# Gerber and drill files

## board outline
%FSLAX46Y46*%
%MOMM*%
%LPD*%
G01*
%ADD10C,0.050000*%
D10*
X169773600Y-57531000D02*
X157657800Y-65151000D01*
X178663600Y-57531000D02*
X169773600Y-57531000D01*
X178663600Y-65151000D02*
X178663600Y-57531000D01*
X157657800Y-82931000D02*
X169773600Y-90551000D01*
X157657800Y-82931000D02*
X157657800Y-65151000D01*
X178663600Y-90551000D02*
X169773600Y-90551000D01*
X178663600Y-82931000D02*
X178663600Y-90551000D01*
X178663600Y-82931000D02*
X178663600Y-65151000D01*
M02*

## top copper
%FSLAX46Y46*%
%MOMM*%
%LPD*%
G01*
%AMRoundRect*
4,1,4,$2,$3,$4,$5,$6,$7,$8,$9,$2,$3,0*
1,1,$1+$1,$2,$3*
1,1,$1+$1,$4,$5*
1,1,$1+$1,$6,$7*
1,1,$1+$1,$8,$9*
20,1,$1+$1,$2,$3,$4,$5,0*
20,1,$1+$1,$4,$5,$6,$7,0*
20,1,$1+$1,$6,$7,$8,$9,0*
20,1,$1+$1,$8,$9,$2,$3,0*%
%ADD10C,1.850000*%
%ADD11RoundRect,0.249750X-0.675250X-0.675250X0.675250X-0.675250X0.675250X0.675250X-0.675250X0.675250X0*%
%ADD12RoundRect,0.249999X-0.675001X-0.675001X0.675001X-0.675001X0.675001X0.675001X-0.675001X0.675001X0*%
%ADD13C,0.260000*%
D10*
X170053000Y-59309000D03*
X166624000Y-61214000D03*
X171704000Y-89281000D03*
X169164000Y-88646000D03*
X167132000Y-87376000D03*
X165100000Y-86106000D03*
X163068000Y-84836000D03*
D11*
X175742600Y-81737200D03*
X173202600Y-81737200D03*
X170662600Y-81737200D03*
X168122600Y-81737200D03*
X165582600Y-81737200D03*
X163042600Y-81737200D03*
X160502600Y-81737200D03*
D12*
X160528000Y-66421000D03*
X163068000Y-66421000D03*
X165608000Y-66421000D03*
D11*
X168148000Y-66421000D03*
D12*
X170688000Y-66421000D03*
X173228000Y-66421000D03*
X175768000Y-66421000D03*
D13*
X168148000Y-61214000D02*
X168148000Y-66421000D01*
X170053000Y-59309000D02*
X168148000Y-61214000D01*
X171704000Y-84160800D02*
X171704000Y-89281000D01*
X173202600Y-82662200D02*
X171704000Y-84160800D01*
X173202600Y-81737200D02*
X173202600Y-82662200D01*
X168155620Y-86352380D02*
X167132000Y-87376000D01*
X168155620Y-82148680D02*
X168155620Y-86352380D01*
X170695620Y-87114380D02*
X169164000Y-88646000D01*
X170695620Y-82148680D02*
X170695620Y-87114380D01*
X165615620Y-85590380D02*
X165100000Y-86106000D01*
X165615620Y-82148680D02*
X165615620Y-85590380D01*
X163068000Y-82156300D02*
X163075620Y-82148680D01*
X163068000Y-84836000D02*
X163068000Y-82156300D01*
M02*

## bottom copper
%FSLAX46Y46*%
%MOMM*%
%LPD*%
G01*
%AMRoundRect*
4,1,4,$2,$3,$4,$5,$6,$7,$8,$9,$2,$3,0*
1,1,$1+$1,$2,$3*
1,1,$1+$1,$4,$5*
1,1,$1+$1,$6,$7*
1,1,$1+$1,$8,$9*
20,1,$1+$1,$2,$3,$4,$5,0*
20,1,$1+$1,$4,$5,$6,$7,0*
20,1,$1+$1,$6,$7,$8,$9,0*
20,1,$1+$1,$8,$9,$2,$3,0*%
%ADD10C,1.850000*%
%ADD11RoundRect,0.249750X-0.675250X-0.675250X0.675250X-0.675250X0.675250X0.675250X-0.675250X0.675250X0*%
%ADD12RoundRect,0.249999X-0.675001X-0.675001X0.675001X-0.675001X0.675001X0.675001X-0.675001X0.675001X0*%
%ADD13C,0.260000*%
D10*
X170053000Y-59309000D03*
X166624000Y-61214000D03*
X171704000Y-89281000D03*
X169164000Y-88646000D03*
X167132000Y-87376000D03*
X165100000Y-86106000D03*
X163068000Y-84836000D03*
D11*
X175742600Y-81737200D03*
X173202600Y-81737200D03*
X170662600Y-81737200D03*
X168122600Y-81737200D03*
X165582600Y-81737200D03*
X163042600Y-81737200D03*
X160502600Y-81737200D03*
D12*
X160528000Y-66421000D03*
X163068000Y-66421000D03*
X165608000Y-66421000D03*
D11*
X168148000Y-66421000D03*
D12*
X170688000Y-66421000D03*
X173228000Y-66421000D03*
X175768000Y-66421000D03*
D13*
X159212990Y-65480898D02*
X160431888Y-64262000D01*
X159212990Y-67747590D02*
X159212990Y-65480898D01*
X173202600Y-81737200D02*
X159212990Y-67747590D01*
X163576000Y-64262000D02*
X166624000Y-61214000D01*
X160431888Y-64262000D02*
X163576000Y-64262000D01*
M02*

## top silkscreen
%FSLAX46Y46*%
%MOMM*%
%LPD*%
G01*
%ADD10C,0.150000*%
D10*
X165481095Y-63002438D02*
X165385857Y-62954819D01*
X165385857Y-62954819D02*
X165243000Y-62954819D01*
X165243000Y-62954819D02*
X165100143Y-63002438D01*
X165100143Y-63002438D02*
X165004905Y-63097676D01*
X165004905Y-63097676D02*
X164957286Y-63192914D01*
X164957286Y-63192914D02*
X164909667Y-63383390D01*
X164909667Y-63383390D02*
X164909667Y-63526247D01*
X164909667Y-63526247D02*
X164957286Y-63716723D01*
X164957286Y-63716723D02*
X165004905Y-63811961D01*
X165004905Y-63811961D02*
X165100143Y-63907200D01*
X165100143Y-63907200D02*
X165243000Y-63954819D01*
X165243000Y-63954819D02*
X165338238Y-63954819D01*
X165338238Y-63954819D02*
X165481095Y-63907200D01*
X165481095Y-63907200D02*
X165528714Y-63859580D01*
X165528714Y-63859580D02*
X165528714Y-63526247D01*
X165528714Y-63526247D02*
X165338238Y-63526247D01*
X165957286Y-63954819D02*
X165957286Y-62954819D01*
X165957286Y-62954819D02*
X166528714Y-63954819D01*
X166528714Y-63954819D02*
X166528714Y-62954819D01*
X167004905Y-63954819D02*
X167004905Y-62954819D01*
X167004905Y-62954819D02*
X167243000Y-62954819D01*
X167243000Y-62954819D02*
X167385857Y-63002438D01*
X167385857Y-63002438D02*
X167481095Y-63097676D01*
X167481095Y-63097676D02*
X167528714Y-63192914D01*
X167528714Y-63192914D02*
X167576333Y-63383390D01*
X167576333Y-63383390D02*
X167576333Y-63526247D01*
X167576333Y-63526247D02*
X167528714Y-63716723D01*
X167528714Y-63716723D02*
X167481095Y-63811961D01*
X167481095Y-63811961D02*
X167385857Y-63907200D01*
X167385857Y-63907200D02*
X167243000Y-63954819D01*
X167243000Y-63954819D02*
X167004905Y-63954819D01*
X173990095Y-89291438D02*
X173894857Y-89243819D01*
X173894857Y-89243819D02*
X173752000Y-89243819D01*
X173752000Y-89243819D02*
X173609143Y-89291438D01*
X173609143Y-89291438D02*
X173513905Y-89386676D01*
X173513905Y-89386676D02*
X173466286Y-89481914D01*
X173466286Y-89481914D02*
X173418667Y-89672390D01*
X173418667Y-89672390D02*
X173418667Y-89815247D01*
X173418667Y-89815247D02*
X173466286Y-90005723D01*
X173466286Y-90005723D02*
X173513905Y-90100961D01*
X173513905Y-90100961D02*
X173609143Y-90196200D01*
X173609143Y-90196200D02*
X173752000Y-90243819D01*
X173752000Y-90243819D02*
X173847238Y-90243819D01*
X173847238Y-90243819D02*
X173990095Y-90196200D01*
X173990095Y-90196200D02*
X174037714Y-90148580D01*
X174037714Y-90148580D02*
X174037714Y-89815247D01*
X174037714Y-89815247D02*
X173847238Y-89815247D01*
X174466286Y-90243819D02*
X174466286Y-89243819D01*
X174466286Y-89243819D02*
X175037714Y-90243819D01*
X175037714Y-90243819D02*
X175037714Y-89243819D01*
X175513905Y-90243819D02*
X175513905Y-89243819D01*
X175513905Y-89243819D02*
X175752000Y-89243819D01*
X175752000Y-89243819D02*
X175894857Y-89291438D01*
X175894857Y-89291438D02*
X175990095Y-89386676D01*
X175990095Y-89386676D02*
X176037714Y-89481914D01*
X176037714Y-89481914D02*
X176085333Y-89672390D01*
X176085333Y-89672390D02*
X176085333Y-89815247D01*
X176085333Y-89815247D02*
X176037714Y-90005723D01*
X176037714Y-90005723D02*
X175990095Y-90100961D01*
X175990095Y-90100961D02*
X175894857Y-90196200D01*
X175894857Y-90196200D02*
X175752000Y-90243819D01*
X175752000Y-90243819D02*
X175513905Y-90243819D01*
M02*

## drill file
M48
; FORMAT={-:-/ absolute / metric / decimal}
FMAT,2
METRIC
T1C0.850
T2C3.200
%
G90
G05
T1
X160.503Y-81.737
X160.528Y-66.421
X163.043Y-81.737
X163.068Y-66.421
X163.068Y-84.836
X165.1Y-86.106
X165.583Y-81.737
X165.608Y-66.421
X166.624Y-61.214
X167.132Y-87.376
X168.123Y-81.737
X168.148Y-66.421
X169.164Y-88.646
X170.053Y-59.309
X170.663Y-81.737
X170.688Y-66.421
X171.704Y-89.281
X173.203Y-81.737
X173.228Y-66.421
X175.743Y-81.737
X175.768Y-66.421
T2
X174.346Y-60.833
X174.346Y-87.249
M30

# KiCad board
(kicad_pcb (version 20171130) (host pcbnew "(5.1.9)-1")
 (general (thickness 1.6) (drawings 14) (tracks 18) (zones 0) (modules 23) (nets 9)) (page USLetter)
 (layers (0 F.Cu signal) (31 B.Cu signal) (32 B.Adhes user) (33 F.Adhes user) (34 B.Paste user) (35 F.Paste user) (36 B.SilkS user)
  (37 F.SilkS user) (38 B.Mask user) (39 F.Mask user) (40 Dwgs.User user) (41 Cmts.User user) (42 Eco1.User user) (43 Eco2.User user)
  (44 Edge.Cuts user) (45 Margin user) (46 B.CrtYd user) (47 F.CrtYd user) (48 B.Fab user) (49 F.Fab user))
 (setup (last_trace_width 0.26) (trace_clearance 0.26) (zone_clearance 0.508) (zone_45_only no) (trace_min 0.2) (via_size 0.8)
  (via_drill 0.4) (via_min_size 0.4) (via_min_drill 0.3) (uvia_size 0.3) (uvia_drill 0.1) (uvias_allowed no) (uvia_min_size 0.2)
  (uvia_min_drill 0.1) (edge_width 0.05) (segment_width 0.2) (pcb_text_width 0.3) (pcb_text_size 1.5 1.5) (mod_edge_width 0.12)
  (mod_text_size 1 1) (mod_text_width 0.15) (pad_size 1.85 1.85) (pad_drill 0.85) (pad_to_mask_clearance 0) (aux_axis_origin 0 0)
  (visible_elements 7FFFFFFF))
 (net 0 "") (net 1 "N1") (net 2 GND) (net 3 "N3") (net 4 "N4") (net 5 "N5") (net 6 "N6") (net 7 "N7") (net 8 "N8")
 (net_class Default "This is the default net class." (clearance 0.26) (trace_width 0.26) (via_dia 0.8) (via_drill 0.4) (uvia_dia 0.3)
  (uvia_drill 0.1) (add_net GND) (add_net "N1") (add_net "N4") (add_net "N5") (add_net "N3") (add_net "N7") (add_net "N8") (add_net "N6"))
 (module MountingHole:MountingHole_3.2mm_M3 (layer F.Cu) (at 174.3456 87.249)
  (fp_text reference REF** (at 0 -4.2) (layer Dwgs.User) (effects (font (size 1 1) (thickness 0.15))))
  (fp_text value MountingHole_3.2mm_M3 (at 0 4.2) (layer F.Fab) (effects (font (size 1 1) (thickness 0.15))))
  (pad 1 np_thru_hole circle (at 0 0) (size 3.2 3.2) (drill 3.2) (layers *.Cu *.Mask)))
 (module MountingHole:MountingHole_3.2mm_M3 (layer F.Cu) (at 174.3456 60.833)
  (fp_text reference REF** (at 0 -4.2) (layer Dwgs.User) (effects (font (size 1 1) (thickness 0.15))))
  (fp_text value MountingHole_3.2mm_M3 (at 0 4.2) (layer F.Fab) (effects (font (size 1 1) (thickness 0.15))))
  (pad 1 np_thru_hole circle (at 0 0) (size 3.2 3.2) (drill 3.2) (layers *.Cu *.Mask)))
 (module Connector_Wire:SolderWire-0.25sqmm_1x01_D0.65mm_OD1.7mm (layer F.Cu) (at 170.053 59.309)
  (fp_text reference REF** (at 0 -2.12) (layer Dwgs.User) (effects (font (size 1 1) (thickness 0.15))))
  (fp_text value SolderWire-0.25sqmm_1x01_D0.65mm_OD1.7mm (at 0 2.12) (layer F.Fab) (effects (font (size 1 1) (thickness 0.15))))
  (pad 1 thru_hole circle (at 0 0) (size 1.85 1.85) (drill 0.85) (layers *.Cu *.Mask) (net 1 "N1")))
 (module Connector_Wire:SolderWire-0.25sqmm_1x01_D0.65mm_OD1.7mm (layer F.Cu) (at 166.624 61.214)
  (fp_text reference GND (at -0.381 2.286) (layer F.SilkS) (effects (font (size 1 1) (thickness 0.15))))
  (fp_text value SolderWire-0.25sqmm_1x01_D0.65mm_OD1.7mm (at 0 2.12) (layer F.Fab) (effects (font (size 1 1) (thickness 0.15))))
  (pad 1 thru_hole circle (at 0 0) (size 1.85 1.85) (drill 0.85) (layers *.Cu *.Mask) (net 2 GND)))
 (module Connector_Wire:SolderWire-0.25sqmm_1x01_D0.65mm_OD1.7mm (layer F.Cu) (at 171.704 89.281)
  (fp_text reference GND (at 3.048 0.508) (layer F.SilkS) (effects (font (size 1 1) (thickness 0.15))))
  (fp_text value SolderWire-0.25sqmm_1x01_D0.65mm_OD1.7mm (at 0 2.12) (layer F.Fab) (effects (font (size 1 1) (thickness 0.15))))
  (pad 1 thru_hole circle (at 0 0) (size 1.85 1.85) (drill 0.85) (layers *.Cu *.Mask) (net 2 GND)))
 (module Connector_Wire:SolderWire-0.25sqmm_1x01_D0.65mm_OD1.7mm (layer F.Cu) (at 169.164 88.646)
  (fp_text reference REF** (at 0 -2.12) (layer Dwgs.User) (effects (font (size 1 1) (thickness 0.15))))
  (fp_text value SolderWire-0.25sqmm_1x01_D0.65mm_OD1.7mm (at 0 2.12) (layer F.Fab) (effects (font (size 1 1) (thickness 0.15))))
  (pad 1 thru_hole circle (at 0 0) (size 1.85 1.85) (drill 0.85) (layers *.Cu *.Mask) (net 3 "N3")))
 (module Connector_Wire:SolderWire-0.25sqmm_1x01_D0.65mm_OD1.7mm (layer F.Cu) (at 167.132 87.376)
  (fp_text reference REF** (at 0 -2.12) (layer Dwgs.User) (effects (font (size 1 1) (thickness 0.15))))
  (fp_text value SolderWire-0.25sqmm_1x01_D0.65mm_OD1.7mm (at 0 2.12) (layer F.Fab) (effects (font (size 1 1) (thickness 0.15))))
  (pad 1 thru_hole circle (at 0 0) (size 1.85 1.85) (drill 0.85) (layers *.Cu *.Mask) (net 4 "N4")))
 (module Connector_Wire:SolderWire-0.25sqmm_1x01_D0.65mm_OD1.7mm (layer F.Cu) (at 165.1 86.106)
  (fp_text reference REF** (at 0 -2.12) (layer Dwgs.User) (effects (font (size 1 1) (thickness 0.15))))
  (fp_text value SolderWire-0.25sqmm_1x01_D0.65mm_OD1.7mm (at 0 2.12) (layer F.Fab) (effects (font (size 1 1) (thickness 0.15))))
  (pad 1 thru_hole circle (at 0 0) (size 1.85 1.85) (drill 0.85) (layers *.Cu *.Mask) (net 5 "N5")))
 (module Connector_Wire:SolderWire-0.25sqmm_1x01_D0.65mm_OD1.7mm (layer F.Cu) (at 163.068 84.836)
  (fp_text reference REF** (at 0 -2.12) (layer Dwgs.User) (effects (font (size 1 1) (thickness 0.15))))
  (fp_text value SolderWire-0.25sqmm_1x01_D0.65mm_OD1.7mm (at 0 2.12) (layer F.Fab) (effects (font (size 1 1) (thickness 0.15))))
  (pad 1 thru_hole circle (at 0 0) (size 1.85 1.85) (drill 0.85) (layers *.Cu *.Mask) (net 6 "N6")))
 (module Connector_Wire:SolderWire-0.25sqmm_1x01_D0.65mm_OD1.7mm (layer F.Cu) (at 175.7426 81.7372)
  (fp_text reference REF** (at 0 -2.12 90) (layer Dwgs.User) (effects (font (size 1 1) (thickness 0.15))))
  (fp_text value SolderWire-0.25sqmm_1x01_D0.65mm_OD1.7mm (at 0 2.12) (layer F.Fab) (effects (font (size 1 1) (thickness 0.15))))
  (pad 1 thru_hole roundrect (at 0 0) (size 1.85 1.85) (drill 0.85) (layers *.Cu *.Mask) (roundrect_rratio 0.135) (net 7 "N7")))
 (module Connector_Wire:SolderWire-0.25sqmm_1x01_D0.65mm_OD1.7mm (layer F.Cu) (at 173.2026 81.7372)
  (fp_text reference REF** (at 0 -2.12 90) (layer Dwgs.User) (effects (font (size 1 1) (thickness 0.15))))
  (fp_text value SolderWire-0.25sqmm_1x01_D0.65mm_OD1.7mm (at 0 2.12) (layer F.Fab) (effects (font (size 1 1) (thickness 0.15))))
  (pad 1 thru_hole roundrect (at 0 0) (size 1.85 1.85) (drill 0.85) (layers *.Cu *.Mask) (roundrect_rratio 0.135) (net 2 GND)))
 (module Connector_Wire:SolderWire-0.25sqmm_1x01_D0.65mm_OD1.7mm (layer F.Cu) (at 170.6626 81.7372)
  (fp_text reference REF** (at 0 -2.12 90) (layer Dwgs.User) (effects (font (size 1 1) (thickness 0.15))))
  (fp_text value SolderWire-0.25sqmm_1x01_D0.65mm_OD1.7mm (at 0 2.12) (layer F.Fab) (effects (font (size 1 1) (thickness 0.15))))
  (pad 1 thru_hole roundrect (at 0 0) (size 1.85 1.85) (drill 0.85) (layers *.Cu *.Mask) (roundrect_rratio 0.135) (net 3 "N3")))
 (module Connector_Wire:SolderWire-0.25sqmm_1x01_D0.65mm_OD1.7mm (layer F.Cu) (at 168.1226 81.7372)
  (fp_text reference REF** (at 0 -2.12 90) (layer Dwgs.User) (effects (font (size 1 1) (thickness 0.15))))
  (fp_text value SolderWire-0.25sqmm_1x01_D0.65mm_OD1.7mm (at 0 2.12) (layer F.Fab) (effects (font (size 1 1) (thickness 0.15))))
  (pad 1 thru_hole roundrect (at 0 0) (size 1.85 1.85) (drill 0.85) (layers *.Cu *.Mask) (roundrect_rratio 0.135) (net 4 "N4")))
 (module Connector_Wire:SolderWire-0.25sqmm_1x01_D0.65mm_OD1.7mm (layer F.Cu) (at 165.5826 81.7372)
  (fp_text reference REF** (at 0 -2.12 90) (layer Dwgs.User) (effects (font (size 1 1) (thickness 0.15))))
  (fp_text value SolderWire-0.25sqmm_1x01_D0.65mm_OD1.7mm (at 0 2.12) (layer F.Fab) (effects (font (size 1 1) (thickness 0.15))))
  (pad 1 thru_hole roundrect (at 0 0) (size 1.85 1.85) (drill 0.85) (layers *.Cu *.Mask) (roundrect_rratio 0.135) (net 5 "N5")))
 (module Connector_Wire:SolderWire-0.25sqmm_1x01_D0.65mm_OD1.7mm (layer F.Cu) (at 163.0426 81.7372)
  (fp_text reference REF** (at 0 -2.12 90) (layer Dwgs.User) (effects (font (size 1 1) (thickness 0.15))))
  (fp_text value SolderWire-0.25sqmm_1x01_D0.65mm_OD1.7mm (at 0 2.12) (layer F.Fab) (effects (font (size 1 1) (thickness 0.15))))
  (pad 1 thru_hole roundrect (at 0 0) (size 1.85 1.85) (drill 0.85) (layers *.Cu *.Mask) (roundrect_rratio 0.135) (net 6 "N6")))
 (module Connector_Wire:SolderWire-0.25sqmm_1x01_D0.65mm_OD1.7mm (layer F.Cu) (at 160.5026 81.7372)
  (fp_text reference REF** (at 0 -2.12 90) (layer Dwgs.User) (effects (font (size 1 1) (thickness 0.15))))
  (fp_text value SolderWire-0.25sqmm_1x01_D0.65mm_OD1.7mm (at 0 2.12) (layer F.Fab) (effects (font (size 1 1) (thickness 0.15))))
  (pad 1 thru_hole roundrect (at 0 0) (size 1.85 1.85) (drill 0.85) (layers *.Cu *.Mask) (roundrect_rratio 0.135) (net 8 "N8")))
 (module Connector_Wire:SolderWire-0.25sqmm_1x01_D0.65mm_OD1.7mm (layer F.Cu) (at 160.528 66.421)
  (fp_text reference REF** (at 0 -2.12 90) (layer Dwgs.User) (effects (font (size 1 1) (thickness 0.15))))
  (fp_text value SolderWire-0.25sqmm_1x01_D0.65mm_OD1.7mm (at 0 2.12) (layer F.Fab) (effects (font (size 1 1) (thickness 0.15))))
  (pad 1 thru_hole roundrect (at 0 0) (size 1.85 1.85) (drill 0.85) (layers *.Cu *.Mask) (roundrect_rratio 0.1351345945945946)))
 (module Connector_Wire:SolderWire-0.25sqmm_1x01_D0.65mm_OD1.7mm (layer F.Cu) (at 163.068 66.421)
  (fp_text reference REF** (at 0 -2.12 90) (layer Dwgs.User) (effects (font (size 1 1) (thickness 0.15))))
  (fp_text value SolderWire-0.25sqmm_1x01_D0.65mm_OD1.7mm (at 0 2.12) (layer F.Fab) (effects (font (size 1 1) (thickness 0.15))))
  (pad 1 thru_hole roundrect (at 0 0) (size 1.85 1.85) (drill 0.85) (layers *.Cu *.Mask) (roundrect_rratio 0.1351345945945946)))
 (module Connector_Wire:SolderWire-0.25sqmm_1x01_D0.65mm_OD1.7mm (layer F.Cu) (at 165.608 66.421)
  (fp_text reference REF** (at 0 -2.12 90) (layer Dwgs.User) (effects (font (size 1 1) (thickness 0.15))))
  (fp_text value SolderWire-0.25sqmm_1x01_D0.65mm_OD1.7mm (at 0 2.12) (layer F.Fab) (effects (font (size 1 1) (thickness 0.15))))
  (pad 1 thru_hole roundrect (at 0 0) (size 1.85 1.85) (drill 0.85) (layers *.Cu *.Mask) (roundrect_rratio 0.1351345945945946)))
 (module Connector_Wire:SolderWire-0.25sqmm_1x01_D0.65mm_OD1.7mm (layer F.Cu) (at 168.148 66.421)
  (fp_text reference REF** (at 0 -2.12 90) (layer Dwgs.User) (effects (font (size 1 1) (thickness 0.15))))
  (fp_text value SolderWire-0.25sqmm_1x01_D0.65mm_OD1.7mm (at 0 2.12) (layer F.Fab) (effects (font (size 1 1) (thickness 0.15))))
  (pad 1 thru_hole roundrect (at 0 0) (size 1.85 1.85) (drill 0.85) (layers *.Cu *.Mask) (roundrect_rratio 0.135) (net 1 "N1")))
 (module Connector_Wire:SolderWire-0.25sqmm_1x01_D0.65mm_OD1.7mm (layer F.Cu) (at 170.688 66.421)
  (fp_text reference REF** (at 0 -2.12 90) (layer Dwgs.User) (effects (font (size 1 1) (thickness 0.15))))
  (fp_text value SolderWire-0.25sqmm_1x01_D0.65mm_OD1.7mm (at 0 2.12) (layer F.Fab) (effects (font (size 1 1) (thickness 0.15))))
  (pad 1 thru_hole roundrect (at 0 0) (size 1.85 1.85) (drill 0.85) (layers *.Cu *.Mask) (roundrect_rratio 0.1351345945945946)))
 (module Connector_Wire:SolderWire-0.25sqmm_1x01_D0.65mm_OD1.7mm (layer F.Cu) (at 173.228 66.421)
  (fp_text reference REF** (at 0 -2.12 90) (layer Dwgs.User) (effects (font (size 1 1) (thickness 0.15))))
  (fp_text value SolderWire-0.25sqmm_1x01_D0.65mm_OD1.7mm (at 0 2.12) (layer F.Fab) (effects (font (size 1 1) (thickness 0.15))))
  (pad 1 thru_hole roundrect (at 0 0) (size 1.85 1.85) (drill 0.85) (layers *.Cu *.Mask) (roundrect_rratio 0.1351345945945946)))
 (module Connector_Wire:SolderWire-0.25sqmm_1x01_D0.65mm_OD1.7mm (layer F.Cu) (at 175.768 66.421)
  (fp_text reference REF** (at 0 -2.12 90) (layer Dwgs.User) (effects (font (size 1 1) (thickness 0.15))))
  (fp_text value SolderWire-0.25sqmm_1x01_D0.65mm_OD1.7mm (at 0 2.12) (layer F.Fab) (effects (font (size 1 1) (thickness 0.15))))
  (pad 1 thru_hole roundrect (at 0 0) (size 1.85 1.85) (drill 0.85) (layers *.Cu *.Mask) (roundrect_rratio 0.1351345945945946)))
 (gr_line (start 169.7736 57.531) (end 157.6578 65.151) (layer Edge.Cuts) (width 0.05))
 (gr_line (start 178.6636 57.531) (end 169.7736 57.531) (layer Edge.Cuts) (width 0.05))
 (gr_line (start 178.6636 65.151) (end 178.6636 57.531) (layer Edge.Cuts) (width 0.05))
 (gr_line (start 157.6578 82.931) (end 169.7736 90.551) (layer Edge.Cuts) (width 0.05))
 (gr_line (start 157.6578 82.931) (end 157.6578 65.151) (layer Edge.Cuts) (width 0.05))
 (gr_line (start 178.6636 90.551) (end 169.7736 90.551) (layer Edge.Cuts) (width 0.05))
 (gr_line (start 178.6636 82.931) (end 178.6636 90.551) (layer Edge.Cuts) (width 0.05))
 (gr_line (start 178.6636 82.931) (end 178.6636 65.151) (layer Edge.Cuts) (width 0.05))
 (segment (start 168.148 61.214) (end 168.148 66.421) (width 0.26) (layer F.Cu) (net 1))
 (segment (start 170.053 59.309) (end 168.148 61.214) (width 0.26) (layer F.Cu) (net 1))
 (segment (start 171.704 84.1608) (end 171.704 89.281) (width 0.26) (layer F.Cu) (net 2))
 (segment (start 173.2026 82.6622) (end 171.704 84.1608) (width 0.26) (layer F.Cu) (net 2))
 (segment (start 173.2026 81.7372) (end 173.2026 82.6622) (width 0.26) (layer F.Cu) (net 2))
 (segment (start 159.21299 65.480898) (end 160.431888 64.262) (width 0.26) (layer B.Cu) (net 2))
 (segment (start 159.21299 67.74759) (end 159.21299 65.480898) (width 0.26) (layer B.Cu) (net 2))
 (segment (start 173.2026 81.7372) (end 159.21299 67.74759) (width 0.26) (layer B.Cu) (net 2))
 (segment (start 163.576 64.262) (end 166.624 61.214) (width 0.26) (layer B.Cu) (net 2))
 (segment (start 160.431888 64.262) (end 163.576 64.262) (width 0.26) (layer B.Cu) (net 2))
 (segment (start 168.15562 86.35238) (end 167.132 87.376) (width 0.26) (layer F.Cu) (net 4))
 (segment (start 168.15562 82.14868) (end 168.15562 86.35238) (width 0.26) (layer F.Cu) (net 4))
 (segment (start 170.69562 87.11438) (end 169.164 88.646) (width 0.26) (layer F.Cu) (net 3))
 (segment (start 170.69562 82.14868) (end 170.69562 87.11438) (width 0.26) (layer F.Cu) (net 3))
 (segment (start 165.61562 85.59038) (end 165.1 86.106) (width 0.26) (layer F.Cu) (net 5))
 (segment (start 165.61562 82.14868) (end 165.61562 85.59038) (width 0.26) (layer F.Cu) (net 5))
 (segment (start 163.068 82.1563) (end 163.07562 82.14868) (width 0.26) (layer F.Cu) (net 6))
 (segment (start 163.068 84.836) (end 163.068 82.1563) (width 0.26) (layer F.Cu) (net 6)))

